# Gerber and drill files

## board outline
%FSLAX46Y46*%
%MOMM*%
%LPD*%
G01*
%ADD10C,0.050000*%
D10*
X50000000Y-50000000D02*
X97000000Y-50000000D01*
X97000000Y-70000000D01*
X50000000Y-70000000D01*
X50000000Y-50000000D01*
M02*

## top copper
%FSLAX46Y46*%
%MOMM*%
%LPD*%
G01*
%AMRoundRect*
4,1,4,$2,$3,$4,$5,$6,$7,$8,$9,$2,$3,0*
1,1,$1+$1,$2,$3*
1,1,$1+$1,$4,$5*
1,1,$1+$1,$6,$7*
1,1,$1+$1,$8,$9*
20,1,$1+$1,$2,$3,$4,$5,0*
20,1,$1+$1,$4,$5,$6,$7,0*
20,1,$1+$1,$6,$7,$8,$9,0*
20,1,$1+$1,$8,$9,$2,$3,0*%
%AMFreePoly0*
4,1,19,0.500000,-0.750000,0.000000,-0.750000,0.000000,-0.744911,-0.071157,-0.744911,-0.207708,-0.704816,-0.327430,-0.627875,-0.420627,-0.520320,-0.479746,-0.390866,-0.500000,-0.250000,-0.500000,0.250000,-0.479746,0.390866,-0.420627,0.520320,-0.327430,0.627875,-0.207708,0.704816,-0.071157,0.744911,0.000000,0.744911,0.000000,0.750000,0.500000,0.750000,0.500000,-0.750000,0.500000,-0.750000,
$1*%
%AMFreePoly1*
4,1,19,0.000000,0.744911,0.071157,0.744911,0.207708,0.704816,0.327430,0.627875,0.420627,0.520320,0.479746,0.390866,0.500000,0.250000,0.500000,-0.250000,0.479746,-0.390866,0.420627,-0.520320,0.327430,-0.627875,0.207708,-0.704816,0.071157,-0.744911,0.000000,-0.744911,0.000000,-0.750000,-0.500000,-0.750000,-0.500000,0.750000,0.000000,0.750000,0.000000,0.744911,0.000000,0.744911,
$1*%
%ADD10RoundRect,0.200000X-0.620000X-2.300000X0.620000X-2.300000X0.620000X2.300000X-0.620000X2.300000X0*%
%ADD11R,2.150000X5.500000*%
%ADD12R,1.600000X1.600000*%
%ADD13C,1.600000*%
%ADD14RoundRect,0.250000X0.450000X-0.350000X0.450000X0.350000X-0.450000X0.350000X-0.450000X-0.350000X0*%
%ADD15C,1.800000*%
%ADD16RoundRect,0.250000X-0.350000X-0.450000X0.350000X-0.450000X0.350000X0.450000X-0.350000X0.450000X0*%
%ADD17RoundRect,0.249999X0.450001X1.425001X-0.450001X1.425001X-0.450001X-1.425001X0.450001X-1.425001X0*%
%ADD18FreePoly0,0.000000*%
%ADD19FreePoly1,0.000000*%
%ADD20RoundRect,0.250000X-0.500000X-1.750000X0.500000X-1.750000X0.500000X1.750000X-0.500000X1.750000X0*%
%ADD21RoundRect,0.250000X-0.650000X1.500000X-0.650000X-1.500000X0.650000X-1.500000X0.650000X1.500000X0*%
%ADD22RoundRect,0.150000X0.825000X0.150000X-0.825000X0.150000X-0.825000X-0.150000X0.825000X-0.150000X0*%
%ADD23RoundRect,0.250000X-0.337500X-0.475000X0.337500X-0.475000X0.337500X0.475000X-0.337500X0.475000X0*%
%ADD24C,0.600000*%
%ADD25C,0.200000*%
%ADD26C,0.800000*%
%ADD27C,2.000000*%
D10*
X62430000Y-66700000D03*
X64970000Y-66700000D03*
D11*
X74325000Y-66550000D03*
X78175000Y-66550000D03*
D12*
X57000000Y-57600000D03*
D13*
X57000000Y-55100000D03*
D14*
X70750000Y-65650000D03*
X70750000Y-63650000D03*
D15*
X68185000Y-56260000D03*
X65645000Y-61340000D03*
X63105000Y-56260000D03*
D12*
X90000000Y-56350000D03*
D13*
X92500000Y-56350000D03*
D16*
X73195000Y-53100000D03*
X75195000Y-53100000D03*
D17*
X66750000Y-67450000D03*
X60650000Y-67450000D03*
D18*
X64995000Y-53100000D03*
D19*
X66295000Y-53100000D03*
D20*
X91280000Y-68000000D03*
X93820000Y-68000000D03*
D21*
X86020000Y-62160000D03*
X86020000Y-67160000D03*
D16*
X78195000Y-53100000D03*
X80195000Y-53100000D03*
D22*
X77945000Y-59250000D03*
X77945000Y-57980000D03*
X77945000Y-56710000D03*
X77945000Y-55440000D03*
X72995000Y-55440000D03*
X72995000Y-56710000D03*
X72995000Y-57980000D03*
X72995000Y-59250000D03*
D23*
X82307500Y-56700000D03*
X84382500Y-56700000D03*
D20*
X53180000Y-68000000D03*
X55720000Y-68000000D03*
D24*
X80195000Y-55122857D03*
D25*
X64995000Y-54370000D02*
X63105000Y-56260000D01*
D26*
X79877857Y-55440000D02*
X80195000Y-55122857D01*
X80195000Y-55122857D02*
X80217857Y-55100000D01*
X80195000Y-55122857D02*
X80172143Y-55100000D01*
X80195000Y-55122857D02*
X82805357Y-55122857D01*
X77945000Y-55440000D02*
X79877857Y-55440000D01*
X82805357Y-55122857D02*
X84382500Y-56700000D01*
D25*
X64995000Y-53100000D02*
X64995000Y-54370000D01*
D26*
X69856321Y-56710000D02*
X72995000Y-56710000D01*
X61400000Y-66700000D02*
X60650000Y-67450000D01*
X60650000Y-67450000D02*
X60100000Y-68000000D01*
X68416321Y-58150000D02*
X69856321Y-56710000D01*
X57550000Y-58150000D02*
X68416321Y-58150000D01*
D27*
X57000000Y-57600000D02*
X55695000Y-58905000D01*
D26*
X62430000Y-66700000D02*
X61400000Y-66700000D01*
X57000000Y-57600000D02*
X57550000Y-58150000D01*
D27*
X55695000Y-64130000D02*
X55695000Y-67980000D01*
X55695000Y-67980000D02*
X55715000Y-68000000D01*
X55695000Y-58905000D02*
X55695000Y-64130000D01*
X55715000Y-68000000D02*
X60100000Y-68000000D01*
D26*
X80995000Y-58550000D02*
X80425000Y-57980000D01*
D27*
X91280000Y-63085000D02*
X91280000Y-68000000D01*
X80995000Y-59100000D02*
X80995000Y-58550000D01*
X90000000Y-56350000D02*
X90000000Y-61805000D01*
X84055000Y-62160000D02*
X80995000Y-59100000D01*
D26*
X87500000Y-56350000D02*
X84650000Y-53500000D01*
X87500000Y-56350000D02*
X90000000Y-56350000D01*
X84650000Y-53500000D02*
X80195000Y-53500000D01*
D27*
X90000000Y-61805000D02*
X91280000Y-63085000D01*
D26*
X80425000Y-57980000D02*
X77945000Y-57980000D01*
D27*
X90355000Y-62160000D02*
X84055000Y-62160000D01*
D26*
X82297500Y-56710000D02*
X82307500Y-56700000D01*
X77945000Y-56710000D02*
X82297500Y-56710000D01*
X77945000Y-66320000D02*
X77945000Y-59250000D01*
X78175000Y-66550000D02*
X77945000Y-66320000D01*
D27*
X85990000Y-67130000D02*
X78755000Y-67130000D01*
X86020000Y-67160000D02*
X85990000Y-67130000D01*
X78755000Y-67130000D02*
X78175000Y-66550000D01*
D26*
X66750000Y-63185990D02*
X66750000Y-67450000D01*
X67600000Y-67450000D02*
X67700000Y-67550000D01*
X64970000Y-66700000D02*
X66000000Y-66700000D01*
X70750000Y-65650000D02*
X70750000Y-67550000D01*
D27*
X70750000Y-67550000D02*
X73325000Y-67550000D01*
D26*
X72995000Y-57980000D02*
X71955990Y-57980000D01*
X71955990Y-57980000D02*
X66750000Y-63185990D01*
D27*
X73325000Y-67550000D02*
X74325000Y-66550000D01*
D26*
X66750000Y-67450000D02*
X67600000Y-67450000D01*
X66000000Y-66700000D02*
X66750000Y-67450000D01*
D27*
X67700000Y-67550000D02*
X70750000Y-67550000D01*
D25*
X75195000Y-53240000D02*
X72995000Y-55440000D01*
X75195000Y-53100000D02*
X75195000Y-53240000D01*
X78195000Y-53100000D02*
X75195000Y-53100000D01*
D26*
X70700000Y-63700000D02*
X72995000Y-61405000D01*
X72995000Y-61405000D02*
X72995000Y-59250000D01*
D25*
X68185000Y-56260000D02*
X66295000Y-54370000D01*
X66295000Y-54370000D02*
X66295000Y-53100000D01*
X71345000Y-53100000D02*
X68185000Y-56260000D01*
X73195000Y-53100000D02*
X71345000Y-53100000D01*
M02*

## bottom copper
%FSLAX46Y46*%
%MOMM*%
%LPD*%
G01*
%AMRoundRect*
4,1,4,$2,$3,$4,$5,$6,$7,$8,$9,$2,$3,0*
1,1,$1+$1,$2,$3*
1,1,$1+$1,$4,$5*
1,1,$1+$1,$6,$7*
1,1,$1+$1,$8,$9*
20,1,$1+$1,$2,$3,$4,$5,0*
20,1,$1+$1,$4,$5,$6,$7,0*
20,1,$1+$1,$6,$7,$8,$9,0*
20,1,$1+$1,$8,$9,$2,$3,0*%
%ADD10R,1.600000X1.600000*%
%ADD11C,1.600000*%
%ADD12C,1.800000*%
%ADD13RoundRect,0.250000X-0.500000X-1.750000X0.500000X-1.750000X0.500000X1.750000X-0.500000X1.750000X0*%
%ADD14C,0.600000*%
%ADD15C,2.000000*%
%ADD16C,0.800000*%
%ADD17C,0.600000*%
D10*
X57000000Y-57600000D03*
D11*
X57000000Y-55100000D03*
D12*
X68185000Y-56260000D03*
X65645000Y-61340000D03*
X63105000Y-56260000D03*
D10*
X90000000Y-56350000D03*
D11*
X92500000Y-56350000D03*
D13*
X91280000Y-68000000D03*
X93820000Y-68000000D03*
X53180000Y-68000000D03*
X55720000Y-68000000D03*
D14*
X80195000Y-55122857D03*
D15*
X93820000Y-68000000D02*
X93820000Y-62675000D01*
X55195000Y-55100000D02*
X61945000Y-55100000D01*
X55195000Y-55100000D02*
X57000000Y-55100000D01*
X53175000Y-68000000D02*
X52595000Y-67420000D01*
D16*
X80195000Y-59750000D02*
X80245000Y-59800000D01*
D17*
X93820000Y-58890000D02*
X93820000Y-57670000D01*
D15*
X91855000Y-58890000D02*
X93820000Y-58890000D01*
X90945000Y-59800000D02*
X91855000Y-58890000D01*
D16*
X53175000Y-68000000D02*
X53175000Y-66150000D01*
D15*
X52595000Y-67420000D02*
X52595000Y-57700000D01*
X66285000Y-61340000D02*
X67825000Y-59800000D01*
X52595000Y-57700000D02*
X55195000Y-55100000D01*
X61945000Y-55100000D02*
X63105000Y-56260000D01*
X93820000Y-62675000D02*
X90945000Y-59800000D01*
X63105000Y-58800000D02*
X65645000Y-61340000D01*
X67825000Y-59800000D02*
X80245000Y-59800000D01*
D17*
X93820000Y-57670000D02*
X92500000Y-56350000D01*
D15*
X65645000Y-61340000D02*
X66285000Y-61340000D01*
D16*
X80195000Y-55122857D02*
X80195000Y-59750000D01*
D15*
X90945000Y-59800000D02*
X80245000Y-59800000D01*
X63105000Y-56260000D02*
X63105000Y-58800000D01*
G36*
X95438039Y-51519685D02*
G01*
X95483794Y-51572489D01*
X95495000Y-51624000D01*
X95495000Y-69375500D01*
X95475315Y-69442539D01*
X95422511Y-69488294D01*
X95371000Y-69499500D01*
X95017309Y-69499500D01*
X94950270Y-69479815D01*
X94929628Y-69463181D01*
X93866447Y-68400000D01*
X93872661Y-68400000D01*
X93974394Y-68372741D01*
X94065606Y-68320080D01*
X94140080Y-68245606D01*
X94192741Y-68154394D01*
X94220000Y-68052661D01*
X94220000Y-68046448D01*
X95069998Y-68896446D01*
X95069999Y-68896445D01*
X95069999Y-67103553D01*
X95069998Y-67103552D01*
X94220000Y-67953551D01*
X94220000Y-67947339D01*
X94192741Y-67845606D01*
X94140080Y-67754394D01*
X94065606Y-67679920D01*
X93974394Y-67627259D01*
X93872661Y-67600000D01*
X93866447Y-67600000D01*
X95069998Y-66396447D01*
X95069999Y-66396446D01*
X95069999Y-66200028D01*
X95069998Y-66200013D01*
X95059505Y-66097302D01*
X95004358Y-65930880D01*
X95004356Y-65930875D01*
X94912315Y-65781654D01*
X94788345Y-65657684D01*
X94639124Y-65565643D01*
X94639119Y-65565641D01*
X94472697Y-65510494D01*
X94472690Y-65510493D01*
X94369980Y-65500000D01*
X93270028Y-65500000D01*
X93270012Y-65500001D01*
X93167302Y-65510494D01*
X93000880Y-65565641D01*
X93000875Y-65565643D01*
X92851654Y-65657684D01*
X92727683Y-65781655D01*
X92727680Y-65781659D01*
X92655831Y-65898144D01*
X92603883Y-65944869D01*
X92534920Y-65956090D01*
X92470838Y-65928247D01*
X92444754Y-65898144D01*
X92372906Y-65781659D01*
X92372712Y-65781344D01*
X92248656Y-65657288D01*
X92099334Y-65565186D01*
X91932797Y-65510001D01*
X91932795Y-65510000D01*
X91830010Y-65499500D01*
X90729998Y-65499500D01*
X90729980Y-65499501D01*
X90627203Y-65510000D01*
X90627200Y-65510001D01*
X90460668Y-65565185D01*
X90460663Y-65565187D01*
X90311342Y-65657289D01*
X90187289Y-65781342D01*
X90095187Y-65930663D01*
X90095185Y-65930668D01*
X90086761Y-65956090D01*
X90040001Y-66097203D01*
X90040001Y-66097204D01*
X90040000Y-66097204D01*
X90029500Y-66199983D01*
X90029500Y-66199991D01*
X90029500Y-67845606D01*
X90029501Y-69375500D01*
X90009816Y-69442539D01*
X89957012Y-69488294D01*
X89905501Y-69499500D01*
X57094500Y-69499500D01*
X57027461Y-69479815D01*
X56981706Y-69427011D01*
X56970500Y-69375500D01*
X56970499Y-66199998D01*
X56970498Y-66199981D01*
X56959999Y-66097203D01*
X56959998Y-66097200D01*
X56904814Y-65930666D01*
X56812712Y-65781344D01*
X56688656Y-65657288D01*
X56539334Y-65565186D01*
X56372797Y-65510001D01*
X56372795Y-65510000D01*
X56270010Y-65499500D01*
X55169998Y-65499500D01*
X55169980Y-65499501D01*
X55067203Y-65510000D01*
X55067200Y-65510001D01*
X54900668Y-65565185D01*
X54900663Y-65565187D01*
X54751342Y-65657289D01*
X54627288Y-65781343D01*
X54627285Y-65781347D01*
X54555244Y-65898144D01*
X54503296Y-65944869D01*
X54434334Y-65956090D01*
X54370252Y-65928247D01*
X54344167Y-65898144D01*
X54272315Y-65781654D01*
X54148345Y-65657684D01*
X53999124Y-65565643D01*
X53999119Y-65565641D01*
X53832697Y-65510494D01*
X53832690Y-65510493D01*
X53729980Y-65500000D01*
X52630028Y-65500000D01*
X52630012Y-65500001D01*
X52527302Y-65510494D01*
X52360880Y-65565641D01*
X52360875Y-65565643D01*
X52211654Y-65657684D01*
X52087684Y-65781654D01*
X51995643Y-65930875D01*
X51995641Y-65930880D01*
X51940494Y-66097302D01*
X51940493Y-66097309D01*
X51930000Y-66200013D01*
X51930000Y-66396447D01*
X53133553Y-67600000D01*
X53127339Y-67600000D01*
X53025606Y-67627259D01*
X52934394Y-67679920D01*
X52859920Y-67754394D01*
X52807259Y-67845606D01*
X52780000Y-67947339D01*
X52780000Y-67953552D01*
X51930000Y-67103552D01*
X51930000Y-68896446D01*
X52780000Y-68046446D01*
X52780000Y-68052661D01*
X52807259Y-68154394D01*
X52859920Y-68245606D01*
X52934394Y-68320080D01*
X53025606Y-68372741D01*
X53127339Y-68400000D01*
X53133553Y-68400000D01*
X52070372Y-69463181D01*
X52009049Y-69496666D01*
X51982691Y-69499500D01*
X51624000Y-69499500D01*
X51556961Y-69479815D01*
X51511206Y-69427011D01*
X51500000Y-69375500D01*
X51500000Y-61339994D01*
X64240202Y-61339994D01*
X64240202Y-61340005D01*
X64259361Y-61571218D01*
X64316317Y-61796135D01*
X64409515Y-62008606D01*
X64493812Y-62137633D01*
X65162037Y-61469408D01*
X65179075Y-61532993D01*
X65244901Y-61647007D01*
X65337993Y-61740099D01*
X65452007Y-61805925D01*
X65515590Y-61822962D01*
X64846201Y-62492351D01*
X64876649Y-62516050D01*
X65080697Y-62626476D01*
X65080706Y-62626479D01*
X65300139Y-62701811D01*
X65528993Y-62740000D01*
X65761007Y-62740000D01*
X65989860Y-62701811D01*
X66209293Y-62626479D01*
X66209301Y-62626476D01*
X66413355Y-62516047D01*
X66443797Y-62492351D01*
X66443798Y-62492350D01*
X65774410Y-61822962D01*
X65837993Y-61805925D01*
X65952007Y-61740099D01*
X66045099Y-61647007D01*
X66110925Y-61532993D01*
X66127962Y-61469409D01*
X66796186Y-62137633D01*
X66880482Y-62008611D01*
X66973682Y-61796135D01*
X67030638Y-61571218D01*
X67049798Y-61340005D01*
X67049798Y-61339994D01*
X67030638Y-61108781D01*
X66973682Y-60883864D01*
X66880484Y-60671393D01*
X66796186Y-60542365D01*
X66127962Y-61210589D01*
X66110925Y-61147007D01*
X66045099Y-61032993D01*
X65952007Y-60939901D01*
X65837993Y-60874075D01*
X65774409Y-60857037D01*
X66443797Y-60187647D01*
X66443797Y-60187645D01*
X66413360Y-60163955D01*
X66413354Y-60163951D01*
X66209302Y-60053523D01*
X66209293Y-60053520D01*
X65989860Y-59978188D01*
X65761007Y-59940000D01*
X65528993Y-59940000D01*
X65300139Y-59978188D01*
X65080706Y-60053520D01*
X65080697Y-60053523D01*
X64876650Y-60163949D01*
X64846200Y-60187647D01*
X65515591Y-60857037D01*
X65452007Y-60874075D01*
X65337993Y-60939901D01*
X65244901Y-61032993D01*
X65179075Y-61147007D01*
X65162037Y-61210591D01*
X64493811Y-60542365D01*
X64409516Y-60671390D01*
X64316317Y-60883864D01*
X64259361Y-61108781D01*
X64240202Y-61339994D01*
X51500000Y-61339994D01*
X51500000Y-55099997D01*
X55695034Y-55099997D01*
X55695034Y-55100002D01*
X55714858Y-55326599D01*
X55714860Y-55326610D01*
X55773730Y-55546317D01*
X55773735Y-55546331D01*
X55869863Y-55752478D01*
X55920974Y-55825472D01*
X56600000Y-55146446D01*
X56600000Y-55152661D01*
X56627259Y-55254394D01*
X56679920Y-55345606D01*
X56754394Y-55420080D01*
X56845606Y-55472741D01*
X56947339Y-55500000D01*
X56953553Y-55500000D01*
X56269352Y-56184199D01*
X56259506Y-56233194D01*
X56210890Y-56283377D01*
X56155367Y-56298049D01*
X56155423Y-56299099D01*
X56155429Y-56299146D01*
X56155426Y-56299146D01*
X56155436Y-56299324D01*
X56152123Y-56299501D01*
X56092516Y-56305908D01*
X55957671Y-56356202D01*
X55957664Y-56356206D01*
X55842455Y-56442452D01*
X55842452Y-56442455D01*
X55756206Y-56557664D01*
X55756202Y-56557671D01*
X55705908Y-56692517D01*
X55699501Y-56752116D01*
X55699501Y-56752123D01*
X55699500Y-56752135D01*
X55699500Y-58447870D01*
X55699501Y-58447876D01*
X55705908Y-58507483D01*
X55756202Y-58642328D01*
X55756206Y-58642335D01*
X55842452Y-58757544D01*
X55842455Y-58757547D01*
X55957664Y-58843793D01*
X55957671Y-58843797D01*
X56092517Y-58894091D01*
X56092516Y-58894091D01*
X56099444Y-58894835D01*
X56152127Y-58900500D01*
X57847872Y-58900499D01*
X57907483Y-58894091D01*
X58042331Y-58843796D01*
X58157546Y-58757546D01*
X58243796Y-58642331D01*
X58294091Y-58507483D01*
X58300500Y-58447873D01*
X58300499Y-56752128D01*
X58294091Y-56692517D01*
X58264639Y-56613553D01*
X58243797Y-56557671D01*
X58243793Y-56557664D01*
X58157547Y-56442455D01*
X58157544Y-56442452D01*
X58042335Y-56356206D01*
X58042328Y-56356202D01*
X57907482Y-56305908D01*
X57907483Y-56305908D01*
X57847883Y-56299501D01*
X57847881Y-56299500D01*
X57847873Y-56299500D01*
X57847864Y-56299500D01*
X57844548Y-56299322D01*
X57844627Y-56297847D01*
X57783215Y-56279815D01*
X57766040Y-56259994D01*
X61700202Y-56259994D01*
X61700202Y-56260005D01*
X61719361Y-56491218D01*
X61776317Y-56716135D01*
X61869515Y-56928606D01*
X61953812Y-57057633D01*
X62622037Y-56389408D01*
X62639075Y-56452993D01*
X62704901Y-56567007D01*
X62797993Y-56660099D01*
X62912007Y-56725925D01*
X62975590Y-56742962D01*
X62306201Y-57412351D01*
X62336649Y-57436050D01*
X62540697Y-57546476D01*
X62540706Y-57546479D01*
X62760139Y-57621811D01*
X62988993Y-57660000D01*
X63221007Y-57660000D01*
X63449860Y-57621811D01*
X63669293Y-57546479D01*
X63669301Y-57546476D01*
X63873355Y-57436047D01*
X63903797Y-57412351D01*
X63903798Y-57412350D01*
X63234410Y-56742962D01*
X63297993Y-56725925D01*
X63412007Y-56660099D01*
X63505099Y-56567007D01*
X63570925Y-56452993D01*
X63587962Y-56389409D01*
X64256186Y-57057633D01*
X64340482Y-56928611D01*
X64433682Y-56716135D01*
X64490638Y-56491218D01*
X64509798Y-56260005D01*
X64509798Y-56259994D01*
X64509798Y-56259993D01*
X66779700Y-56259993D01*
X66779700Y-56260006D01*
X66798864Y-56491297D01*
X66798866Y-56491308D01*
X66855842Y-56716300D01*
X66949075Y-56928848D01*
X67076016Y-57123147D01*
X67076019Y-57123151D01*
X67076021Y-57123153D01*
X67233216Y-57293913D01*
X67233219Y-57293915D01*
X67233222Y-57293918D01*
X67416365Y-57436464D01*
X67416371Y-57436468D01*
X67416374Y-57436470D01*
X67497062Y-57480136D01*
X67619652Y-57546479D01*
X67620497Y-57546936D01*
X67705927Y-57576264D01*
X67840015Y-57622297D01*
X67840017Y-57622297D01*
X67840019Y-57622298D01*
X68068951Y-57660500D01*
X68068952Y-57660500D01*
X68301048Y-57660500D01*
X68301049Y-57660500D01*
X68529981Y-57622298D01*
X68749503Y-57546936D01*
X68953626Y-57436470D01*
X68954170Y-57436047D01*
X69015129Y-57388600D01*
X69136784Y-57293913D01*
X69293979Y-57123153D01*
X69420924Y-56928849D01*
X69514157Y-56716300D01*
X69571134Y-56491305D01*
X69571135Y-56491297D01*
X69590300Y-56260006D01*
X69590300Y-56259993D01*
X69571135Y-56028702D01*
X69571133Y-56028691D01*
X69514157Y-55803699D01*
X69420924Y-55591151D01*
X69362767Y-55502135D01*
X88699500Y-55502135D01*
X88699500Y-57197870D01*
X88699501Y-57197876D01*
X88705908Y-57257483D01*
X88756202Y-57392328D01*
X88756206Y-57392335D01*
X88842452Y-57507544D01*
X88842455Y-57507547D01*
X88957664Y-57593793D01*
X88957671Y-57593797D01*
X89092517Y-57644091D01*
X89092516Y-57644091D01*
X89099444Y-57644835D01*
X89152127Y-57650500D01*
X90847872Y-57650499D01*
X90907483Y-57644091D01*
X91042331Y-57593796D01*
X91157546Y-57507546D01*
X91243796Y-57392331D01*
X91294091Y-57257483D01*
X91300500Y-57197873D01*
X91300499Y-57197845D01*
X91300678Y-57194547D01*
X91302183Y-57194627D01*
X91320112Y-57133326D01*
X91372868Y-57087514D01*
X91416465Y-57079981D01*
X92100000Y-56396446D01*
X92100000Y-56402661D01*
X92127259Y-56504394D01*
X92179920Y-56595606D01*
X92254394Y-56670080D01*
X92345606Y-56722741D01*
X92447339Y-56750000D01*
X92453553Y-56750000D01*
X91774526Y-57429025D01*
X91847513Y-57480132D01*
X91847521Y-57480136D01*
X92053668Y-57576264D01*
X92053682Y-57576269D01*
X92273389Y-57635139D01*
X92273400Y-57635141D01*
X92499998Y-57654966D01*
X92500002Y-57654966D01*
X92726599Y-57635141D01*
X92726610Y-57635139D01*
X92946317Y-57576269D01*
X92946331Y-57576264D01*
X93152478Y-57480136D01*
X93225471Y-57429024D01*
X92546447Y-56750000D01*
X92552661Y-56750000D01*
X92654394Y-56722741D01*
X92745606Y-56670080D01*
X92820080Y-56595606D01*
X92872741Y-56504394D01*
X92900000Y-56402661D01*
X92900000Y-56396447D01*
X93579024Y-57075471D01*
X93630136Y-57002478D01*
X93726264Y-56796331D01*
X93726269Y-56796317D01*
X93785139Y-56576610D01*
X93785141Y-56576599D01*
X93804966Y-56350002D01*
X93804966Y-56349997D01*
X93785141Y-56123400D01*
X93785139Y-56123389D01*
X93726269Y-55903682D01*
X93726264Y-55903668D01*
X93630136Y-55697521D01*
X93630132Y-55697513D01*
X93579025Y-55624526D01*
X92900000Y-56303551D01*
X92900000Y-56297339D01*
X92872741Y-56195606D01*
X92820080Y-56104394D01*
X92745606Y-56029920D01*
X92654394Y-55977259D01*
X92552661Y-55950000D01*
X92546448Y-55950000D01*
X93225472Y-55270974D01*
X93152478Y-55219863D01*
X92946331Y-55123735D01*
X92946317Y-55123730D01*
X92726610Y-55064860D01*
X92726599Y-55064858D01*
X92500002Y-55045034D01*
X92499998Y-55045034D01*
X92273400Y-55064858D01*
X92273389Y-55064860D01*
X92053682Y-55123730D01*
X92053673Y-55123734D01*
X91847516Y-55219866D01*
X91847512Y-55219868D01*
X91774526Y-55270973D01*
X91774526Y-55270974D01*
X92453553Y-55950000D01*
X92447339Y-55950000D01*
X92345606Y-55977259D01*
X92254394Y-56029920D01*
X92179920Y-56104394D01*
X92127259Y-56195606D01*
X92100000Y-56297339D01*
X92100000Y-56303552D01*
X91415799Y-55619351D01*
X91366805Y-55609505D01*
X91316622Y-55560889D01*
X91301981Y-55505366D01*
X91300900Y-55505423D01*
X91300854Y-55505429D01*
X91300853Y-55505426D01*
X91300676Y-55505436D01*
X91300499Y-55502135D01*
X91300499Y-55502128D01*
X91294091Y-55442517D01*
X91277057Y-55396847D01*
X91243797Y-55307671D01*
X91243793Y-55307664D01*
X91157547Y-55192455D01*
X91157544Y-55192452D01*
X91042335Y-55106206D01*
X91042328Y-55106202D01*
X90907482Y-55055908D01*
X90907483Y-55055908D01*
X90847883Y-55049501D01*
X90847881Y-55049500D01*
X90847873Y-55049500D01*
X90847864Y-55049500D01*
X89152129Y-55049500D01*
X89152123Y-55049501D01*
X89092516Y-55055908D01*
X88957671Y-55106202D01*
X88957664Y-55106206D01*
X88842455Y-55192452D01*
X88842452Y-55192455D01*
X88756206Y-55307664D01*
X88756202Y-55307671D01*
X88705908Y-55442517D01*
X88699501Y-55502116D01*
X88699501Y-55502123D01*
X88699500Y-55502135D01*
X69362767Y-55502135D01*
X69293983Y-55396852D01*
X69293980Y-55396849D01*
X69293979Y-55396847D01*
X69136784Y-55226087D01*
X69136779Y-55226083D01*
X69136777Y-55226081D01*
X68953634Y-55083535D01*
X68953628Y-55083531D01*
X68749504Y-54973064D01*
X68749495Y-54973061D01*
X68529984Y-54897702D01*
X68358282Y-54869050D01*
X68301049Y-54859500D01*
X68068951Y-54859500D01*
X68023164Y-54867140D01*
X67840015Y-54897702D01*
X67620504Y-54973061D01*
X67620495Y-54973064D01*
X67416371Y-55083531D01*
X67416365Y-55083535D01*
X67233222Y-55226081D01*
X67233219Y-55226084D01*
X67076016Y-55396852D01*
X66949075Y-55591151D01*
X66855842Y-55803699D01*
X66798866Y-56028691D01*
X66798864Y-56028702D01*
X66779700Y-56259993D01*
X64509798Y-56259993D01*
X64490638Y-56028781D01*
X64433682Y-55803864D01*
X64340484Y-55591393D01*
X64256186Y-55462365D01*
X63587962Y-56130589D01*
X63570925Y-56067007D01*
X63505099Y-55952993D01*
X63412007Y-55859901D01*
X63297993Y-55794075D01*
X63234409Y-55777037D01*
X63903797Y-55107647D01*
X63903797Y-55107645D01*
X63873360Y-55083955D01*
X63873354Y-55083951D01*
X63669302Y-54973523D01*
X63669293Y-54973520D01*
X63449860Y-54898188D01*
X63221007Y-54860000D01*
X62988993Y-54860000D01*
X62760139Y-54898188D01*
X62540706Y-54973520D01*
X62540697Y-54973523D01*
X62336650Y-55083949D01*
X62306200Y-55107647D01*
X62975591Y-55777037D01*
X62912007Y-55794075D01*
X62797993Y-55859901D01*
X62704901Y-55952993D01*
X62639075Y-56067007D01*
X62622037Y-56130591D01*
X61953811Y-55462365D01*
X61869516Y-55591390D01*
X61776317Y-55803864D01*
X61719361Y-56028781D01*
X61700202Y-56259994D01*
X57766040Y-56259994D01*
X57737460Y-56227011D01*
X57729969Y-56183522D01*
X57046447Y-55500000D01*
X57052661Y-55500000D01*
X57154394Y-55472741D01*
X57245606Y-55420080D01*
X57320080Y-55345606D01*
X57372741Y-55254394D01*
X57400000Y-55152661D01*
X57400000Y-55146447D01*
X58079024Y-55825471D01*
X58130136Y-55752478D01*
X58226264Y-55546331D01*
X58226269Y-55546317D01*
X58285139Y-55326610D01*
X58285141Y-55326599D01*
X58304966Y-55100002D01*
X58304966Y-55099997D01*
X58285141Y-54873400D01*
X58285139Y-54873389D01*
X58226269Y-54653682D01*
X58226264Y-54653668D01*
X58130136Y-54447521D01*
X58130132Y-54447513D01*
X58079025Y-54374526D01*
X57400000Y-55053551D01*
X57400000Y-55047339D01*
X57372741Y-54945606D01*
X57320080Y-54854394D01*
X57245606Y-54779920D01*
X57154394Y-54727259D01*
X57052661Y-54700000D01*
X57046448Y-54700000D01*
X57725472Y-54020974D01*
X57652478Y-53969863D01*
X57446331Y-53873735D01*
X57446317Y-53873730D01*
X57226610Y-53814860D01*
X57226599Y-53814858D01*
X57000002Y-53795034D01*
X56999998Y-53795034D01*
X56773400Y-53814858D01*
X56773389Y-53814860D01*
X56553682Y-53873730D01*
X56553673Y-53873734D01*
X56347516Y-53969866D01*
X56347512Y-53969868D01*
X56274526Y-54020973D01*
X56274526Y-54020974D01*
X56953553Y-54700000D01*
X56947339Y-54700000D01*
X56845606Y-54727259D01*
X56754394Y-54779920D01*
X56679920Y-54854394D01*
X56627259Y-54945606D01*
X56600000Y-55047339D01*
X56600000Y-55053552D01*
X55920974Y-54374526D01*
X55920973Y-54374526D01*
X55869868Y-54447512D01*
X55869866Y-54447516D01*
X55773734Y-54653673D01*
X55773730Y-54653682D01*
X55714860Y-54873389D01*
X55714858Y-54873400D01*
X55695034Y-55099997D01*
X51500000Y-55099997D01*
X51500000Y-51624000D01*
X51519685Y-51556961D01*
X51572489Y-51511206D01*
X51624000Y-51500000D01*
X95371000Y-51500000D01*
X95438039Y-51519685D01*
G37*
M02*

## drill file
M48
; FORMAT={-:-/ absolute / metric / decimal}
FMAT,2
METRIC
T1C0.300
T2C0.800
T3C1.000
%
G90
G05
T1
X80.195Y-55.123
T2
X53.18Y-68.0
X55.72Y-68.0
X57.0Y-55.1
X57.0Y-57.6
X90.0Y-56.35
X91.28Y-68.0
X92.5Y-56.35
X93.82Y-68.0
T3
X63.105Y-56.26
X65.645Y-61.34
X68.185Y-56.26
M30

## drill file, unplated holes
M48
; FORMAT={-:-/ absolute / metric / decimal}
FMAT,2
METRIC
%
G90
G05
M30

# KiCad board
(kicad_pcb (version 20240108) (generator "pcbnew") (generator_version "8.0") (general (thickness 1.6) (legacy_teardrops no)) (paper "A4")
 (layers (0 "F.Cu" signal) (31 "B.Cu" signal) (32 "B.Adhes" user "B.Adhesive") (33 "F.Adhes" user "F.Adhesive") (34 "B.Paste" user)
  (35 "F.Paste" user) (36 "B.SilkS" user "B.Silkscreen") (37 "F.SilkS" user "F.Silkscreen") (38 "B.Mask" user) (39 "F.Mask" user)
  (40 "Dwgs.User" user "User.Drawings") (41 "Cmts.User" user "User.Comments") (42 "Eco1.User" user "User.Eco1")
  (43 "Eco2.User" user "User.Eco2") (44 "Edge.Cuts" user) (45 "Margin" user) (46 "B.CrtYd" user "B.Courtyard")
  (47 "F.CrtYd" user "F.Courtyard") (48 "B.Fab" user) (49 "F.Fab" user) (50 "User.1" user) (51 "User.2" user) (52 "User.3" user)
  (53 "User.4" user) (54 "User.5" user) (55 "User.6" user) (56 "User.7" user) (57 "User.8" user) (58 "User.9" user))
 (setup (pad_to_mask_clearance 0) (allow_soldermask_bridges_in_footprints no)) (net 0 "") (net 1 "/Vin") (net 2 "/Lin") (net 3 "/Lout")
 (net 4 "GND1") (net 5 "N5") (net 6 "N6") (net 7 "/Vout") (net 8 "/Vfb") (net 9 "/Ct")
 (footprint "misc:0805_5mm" (layer "F.Cu") (at 63.7 66.7)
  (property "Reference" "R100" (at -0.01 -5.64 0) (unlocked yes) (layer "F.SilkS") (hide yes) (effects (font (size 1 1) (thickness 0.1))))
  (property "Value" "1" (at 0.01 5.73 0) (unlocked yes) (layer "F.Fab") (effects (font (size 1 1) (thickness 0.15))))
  (pad "1" smd roundrect (at -1.27 0) (size 1.64 5) (layers "F.Cu" "F.Paste" "F.Mask") (roundrect_rratio 0.1219512195) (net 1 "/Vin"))
  (pad "2" smd roundrect (at 1.27 0) (size 1.64 5) (layers "F.Cu" "F.Paste" "F.Mask") (roundrect_rratio 0.1219512195) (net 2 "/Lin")))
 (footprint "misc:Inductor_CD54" (layer "F.Cu") (at 76.25 66.55 90)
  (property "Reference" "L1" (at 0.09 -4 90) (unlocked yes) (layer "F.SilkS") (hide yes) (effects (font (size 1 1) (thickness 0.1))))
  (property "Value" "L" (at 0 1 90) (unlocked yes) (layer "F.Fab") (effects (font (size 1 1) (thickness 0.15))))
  (pad "1" smd rect (at 0 -1.925 90) (size 5.5 2.15) (layers "F.Cu" "F.Paste" "F.Mask") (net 2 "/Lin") (thermal_bridge_angle 45))
  (pad "2" smd rect (at 0 1.925 90) (size 5.5 2.15) (layers "F.Cu" "F.Paste" "F.Mask") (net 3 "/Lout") (thermal_bridge_angle 45)))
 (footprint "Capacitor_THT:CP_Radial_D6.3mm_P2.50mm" (layer "F.Cu") (at 57 57.6 90)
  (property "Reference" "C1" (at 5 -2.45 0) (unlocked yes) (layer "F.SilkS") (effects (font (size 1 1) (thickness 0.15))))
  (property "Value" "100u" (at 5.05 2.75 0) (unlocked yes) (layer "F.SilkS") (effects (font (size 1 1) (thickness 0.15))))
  (pad "1" thru_hole rect (at 0 0 90) (size 1.6 1.6) (drill 0.8) (layers "*.Cu" "*.Mask") (remove_unused_layers no) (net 1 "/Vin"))
  (pad "2" thru_hole circle (at 2.5 0 90) (size 1.6 1.6) (drill 0.8) (layers "*.Cu" "*.Mask") (remove_unused_layers no) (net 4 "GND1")))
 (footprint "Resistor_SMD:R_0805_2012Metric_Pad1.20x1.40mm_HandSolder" (layer "F.Cu") (at 70.75 64.65 90)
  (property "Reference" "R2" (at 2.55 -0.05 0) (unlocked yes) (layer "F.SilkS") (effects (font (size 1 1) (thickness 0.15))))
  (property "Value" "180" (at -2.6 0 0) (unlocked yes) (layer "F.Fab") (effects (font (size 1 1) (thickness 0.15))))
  (pad "1" smd roundrect (at -1 0 90) (size 1.2 1.4) (layers "F.Cu" "F.Paste" "F.Mask") (roundrect_rratio 0.208333) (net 2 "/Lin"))
  (pad "2" smd roundrect (at 1 0 90) (size 1.2 1.4) (layers "F.Cu" "F.Paste" "F.Mask") (roundrect_rratio 0.208333) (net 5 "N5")))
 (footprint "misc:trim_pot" (layer "F.Cu") (at 65.645 58.8 180)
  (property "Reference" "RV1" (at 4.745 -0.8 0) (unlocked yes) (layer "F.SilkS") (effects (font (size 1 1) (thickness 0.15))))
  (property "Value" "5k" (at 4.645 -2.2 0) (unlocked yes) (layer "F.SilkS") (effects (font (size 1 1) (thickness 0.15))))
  (pad "1" thru_hole circle (at -2.54 2.54 180) (size 1.8 1.8) (drill 1) (layers "*.Cu" "*.Mask") (remove_unused_layers no) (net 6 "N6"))
  (pad "2" thru_hole circle (at 0 -2.54 180) (size 1.8 1.8) (drill 1) (layers "*.Cu" "*.Mask") (remove_unused_layers no) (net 4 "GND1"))
  (pad "3" thru_hole circle (at 2.54 2.54 180) (size 1.8 1.8) (drill 1) (layers "*.Cu" "*.Mask") (remove_unused_layers no) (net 4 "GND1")))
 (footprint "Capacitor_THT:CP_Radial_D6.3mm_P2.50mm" (layer "F.Cu") (at 90 56.35)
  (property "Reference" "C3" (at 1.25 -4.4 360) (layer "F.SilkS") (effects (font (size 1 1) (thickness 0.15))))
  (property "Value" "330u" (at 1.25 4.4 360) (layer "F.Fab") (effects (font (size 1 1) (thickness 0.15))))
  (pad "1" thru_hole rect (at 0 0) (size 1.6 1.6) (drill 0.8) (layers "*.Cu" "*.Mask") (remove_unused_layers no) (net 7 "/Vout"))
  (pad "2" thru_hole circle (at 2.5 0) (size 1.6 1.6) (drill 0.8) (layers "*.Cu" "*.Mask") (remove_unused_layers no) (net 4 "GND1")))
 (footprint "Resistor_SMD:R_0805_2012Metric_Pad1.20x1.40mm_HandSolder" (layer "F.Cu") (at 74.195 53.1)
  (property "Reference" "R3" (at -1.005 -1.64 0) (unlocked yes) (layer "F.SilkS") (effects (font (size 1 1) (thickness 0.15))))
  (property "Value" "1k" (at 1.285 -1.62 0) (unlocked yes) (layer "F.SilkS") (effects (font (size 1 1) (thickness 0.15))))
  (pad "1" smd roundrect (at -1 0) (size 1.2 1.4) (layers "F.Cu" "F.Paste" "F.Mask") (roundrect_rratio 0.208333) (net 6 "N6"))
  (pad "2" smd roundrect (at 1 0) (size 1.2 1.4) (layers "F.Cu" "F.Paste" "F.Mask") (roundrect_rratio 0.208333) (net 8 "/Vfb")))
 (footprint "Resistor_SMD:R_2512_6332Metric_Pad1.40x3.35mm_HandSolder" (layer "F.Cu") (at 63.7 67.45 180)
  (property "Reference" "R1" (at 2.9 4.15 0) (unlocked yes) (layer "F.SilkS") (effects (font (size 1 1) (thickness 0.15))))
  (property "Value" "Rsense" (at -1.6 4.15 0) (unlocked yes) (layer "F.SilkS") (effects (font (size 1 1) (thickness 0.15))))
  (pad "1" smd roundrect (at -3.05 0 180) (size 1.4 3.35) (layers "F.Cu" "F.Paste" "F.Mask") (roundrect_rratio 0.178571) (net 2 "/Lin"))
  (pad "2" smd roundrect (at 3.05 0 180) (size 1.4 3.35) (layers "F.Cu" "F.Paste" "F.Mask") (roundrect_rratio 0.178571) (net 1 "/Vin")))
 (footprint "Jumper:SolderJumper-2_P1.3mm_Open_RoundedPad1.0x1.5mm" (layer "F.Cu") (at 65.645 53.1)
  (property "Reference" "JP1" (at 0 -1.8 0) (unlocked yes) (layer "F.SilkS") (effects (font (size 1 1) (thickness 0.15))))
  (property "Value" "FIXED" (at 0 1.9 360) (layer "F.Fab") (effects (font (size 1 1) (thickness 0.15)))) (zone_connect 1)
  (pad "1" smd custom (at -0.65 0) (size 1 0.5) (layers "F.Cu" "F.Mask") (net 4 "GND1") (zone_connect 2) (thermal_bridge_angle 45)
   (options (clearance outline) (anchor rect)) (primitives))
  (pad "2" smd custom (at 0.65 0) (size 1 0.5) (layers "F.Cu" "F.Mask") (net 6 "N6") (zone_connect 2) (thermal_bridge_angle 45)
   (options (clearance outline) (anchor rect)) (primitives)))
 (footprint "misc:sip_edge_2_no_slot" (layer "F.Cu") (at 92.55 70)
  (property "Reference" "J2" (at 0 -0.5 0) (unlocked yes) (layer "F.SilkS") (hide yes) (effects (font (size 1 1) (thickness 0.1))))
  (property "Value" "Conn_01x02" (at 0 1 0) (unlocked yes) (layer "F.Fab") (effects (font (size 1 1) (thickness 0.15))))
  (pad "1" thru_hole roundrect (at -1.27 -2) (size 1.5 4) (drill 0.8) (layers "*.Cu" "*.Mask") (remove_unused_layers no)
   (roundrect_rratio 0.1666666667) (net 7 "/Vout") (thermal_bridge_angle 45))
  (pad "2" thru_hole roundrect (at 1.27 -2) (size 1.5 4) (drill 0.8) (layers "*.Cu" "*.Mask") (remove_unused_layers no)
   (roundrect_rratio 0.1666666667) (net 4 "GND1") (thermal_bridge_angle 45)))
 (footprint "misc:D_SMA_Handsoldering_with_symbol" (layer "F.Cu") (at 86.02 64.66 -90)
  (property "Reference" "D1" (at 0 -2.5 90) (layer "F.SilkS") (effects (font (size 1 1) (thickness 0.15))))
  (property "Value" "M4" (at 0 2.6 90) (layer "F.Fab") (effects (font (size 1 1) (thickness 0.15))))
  (pad "1" smd roundrect (at -2.5 0 270) (size 3.5 1.8) (layers "F.Cu" "F.Paste" "F.Mask") (roundrect_rratio 0.1388888889) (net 7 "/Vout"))
  (pad "2" smd roundrect (at 2.5 0 270) (size 3.5 1.8) (layers "F.Cu" "F.Paste" "F.Mask") (roundrect_rratio 0.1388888889) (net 3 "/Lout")))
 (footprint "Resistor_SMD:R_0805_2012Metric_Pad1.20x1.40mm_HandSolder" (layer "F.Cu") (at 79.195 53.1)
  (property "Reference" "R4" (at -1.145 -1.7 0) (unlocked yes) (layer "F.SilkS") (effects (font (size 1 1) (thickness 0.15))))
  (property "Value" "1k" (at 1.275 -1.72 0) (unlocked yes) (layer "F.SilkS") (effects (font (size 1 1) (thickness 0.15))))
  (pad "1" smd roundrect (at -1 0) (size 1.2 1.4) (layers "F.Cu" "F.Paste" "F.Mask") (roundrect_rratio 0.208333) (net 8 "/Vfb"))
  (pad "2" smd roundrect (at 1 0) (size 1.2 1.4) (layers "F.Cu" "F.Paste" "F.Mask") (roundrect_rratio 0.208333) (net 7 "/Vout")))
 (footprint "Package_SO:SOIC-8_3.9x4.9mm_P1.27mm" (layer "F.Cu") (at 75.47 57.345 180)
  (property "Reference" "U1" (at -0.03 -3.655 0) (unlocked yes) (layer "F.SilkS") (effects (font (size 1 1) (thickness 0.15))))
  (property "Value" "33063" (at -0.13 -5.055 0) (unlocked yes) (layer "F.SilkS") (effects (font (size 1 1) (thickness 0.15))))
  (pad "1" smd roundrect (at -2.475 -1.905 180) (size 1.95 0.6) (layers "F.Cu" "F.Paste" "F.Mask") (roundrect_rratio 0.25) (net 3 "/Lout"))
  (pad "2" smd roundrect (at -2.475 -0.635 180) (size 1.95 0.6) (layers "F.Cu" "F.Paste" "F.Mask") (roundrect_rratio 0.25) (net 7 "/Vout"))
  (pad "3" smd roundrect (at -2.475 0.635 180) (size 1.95 0.6) (layers "F.Cu" "F.Paste" "F.Mask") (roundrect_rratio 0.25) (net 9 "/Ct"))
  (pad "4" smd roundrect (at -2.475 1.905 180) (size 1.95 0.6) (layers "F.Cu" "F.Paste" "F.Mask") (roundrect_rratio 0.25) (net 4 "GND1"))
  (pad "5" smd roundrect (at 2.475 1.905 180) (size 1.95 0.6) (layers "F.Cu" "F.Paste" "F.Mask") (roundrect_rratio 0.25) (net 8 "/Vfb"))
  (pad "6" smd roundrect (at 2.475 0.635 180) (size 1.95 0.6) (layers "F.Cu" "F.Paste" "F.Mask") (roundrect_rratio 0.25) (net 1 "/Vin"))
  (pad "7" smd roundrect (at 2.475 -0.635 180) (size 1.95 0.6) (layers "F.Cu" "F.Paste" "F.Mask") (roundrect_rratio 0.25) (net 2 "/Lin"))
  (pad "8" smd roundrect (at 2.475 -1.905 180) (size 1.95 0.6) (layers "F.Cu" "F.Paste" "F.Mask") (roundrect_rratio 0.25) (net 5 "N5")))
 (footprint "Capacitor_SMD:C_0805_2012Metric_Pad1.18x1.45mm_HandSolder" (layer "F.Cu") (at 83.345 56.7)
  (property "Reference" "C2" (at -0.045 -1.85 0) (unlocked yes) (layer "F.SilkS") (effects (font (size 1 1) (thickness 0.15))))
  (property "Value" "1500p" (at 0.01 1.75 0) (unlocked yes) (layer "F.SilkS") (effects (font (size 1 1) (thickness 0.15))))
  (pad "1" smd roundrect (at -1.0375 0) (size 1.175 1.45) (layers "F.Cu" "F.Paste" "F.Mask") (roundrect_rratio 0.212766) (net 9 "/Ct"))
  (pad "2" smd roundrect (at 1.0375 0) (size 1.175 1.45) (layers "F.Cu" "F.Paste" "F.Mask") (roundrect_rratio 0.212766) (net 4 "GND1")))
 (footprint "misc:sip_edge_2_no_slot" (layer "F.Cu") (at 54.45 70)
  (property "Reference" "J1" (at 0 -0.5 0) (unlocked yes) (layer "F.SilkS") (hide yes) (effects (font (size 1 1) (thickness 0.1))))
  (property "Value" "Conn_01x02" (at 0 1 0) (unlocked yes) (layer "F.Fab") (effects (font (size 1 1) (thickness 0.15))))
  (pad "1" thru_hole roundrect (at -1.27 -2) (size 1.5 4) (drill 0.8) (layers "*.Cu" "*.Mask") (remove_unused_layers no)
   (roundrect_rratio 0.1666666667) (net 4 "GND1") (thermal_bridge_angle 45))
  (pad "2" thru_hole roundrect (at 1.27 -2) (size 1.5 4) (drill 0.8) (layers "*.Cu" "*.Mask") (remove_unused_layers no)
   (roundrect_rratio 0.1666666667) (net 1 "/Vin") (thermal_bridge_angle 45)))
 (gr_rect (start 50 50) (end 97 70) (stroke (width 0.05) (type default)) (fill none) (layer "Edge.Cuts"))
 (segment (start 70.7 63.7) (end 72.995 61.405) (width 0.8) (layer "F.Cu") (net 5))
 (segment (start 72.995 61.405) (end 72.995 59.25) (width 0.8) (layer "F.Cu") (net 5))
 (segment (start 64.995 54.37) (end 63.105 56.26) (width 0.2) (layer "F.Cu") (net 4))
 (segment (start 79.877857 55.44) (end 80.195 55.122857) (width 0.8) (layer "F.Cu") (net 4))
 (segment (start 80.195 55.122857) (end 80.217857 55.1) (width 0.8) (layer "F.Cu") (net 4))
 (segment (start 80.195 55.122857) (end 80.172143 55.1) (width 0.8) (layer "F.Cu") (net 4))
 (segment (start 80.195 55.122857) (end 82.805357 55.122857) (width 0.8) (layer "F.Cu") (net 4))
 (segment (start 77.945 55.44) (end 79.877857 55.44) (width 0.8) (layer "F.Cu") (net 4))
 (segment (start 82.805357 55.122857) (end 84.3825 56.7) (width 0.8) (layer "F.Cu") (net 4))
 (segment (start 64.995 53.1) (end 64.995 54.37) (width 0.2) (layer "F.Cu") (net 4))
 (via (at 80.195 55.122857) (size 0.6) (drill 0.3) (layers "F.Cu" "B.Cu") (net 4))
 (segment (start 93.82 68) (end 93.82 62.675) (width 2) (layer "B.Cu") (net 4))
 (segment (start 55.195 55.1) (end 61.945 55.1) (width 2) (layer "B.Cu") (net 4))
 (segment (start 55.195 55.1) (end 57 55.1) (width 2) (layer "B.Cu") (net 4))
 (segment (start 53.175 68) (end 52.595 67.42) (width 2) (layer "B.Cu") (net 4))
 (segment (start 80.195 59.75) (end 80.245 59.8) (width 0.8) (layer "B.Cu") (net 4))
 (segment (start 93.82 58.89) (end 93.82 57.67) (width 0.6) (layer "B.Cu") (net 4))
 (segment (start 91.855 58.89) (end 93.82 58.89) (width 2) (layer "B.Cu") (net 4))
 (segment (start 90.945 59.8) (end 91.855 58.89) (width 2) (layer "B.Cu") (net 4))
 (segment (start 53.175 68) (end 53.175 66.15) (width 0.8) (layer "B.Cu") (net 4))
 (segment (start 52.595 67.42) (end 52.595 57.7) (width 2) (layer "B.Cu") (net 4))
 (segment (start 66.285 61.34) (end 67.825 59.8) (width 2) (layer "B.Cu") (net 4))
 (segment (start 52.595 57.7) (end 55.195 55.1) (width 2) (layer "B.Cu") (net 4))
 (segment (start 61.945 55.1) (end 63.105 56.26) (width 2) (layer "B.Cu") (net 4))
 (segment (start 93.82 62.675) (end 90.945 59.8) (width 2) (layer "B.Cu") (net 4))
 (segment (start 63.105 58.8) (end 65.645 61.34) (width 2) (layer "B.Cu") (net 4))
 (segment (start 67.825 59.8) (end 80.245 59.8) (width 2) (layer "B.Cu") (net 4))
 (segment (start 93.82 57.67) (end 92.5 56.35) (width 0.6) (layer "B.Cu") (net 4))
 (segment (start 65.645 61.34) (end 66.285 61.34) (width 2) (layer "B.Cu") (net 4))
 (segment (start 80.195 55.122857) (end 80.195 59.75) (width 0.8) (layer "B.Cu") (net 4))
 (segment (start 90.945 59.8) (end 80.245 59.8) (width 2) (layer "B.Cu") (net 4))
 (segment (start 63.105 56.26) (end 63.105 58.8) (width 2) (layer "B.Cu") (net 4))
 (segment (start 69.856321 56.71) (end 72.995 56.71) (width 0.8) (layer "F.Cu") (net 1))
 (segment (start 61.4 66.7) (end 60.65 67.45) (width 0.8) (layer "F.Cu") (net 1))
 (segment (start 60.65 67.45) (end 60.1 68) (width 0.8) (layer "F.Cu") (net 1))
 (segment (start 68.416321 58.15) (end 69.856321 56.71) (width 0.8) (layer "F.Cu") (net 1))
 (segment (start 57.55 58.15) (end 68.416321 58.15) (width 0.8) (layer "F.Cu") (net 1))
 (segment (start 57 57.6) (end 55.695 58.905) (width 2) (layer "F.Cu") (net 1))
 (segment (start 62.43 66.7) (end 61.4 66.7) (width 0.8) (layer "F.Cu") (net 1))
 (segment (start 57 57.6) (end 57.55 58.15) (width 0.8) (layer "F.Cu") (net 1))
 (segment (start 55.695 64.13) (end 55.695 67.98) (width 2) (layer "F.Cu") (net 1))
 (segment (start 55.695 67.98) (end 55.715 68) (width 2) (layer "F.Cu") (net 1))
 (segment (start 55.695 58.905) (end 55.695 64.13) (width 2) (layer "F.Cu") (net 1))
 (segment (start 55.715 68) (end 60.1 68) (width 2) (layer "F.Cu") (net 1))
 (segment (start 80.995 58.55) (end 80.425 57.98) (width 0.8) (layer "F.Cu") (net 7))
 (segment (start 91.28 63.085) (end 91.28 68) (width 2) (layer "F.Cu") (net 7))
 (segment (start 80.995 59.1) (end 80.995 58.55) (width 2) (layer "F.Cu") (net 7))
 (segment (start 90 56.35) (end 90 61.805) (width 2) (layer "F.Cu") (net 7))
 (segment (start 84.055 62.16) (end 80.995 59.1) (width 2) (layer "F.Cu") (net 7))
 (segment (start 87.5 56.35) (end 84.65 53.5) (width 0.8) (layer "F.Cu") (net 7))
 (segment (start 87.5 56.35) (end 90 56.35) (width 0.8) (layer "F.Cu") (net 7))
 (segment (start 84.65 53.5) (end 80.195 53.5) (width 0.8) (layer "F.Cu") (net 7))
 (segment (start 90 61.805) (end 91.28 63.085) (width 2) (layer "F.Cu") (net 7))
 (segment (start 80.425 57.98) (end 77.945 57.98) (width 0.8) (layer "F.Cu") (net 7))
 (segment (start 90.355 62.16) (end 84.055 62.16) (width 2) (layer "F.Cu") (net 7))
 (segment (start 82.2975 56.71) (end 82.3075 56.7) (width 0.8) (layer "F.Cu") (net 9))
 (segment (start 77.945 56.71) (end 82.2975 56.71) (width 0.8) (layer "F.Cu") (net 9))
 (segment (start 77.945 66.32) (end 77.945 59.25) (width 0.8) (layer "F.Cu") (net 3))
 (segment (start 78.175 66.55) (end 77.945 66.32) (width 0.8) (layer "F.Cu") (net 3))
 (segment (start 85.99 67.13) (end 78.755 67.13) (width 2) (layer "F.Cu") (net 3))
 (segment (start 86.02 67.16) (end 85.99 67.13) (width 2) (layer "F.Cu") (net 3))
 (segment (start 78.755 67.13) (end 78.175 66.55) (width 2) (layer "F.Cu") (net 3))
 (segment (start 66.75 63.18599) (end 66.75 67.45) (width 0.8) (layer "F.Cu") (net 2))
 (segment (start 67.6 67.45) (end 67.7 67.55) (width 0.8) (layer "F.Cu") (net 2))
 (segment (start 64.97 66.7) (end 66 66.7) (width 0.8) (layer "F.Cu") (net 2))
 (segment (start 70.75 65.65) (end 70.75 67.55) (width 0.8) (layer "F.Cu") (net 2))
 (segment (start 70.75 67.55) (end 73.325 67.55) (width 2) (layer "F.Cu") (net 2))
 (segment (start 72.995 57.98) (end 71.95599 57.98) (width 0.8) (layer "F.Cu") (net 2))
 (segment (start 71.95599 57.98) (end 66.75 63.18599) (width 0.8) (layer "F.Cu") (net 2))
 (segment (start 73.325 67.55) (end 74.325 66.55) (width 2) (layer "F.Cu") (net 2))
 (segment (start 66.75 67.45) (end 67.6 67.45) (width 0.8) (layer "F.Cu") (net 2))
 (segment (start 66 66.7) (end 66.75 67.45) (width 0.8) (layer "F.Cu") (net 2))
 (segment (start 67.7 67.55) (end 70.75 67.55) (width 2) (layer "F.Cu") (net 2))
 (segment (start 75.195 53.24) (end 72.995 55.44) (width 0.2) (layer "F.Cu") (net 8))
 (segment (start 75.195 53.1) (end 75.195 53.24) (width 0.2) (layer "F.Cu") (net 8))
 (segment (start 78.195 53.1) (end 75.195 53.1) (width 0.2) (layer "F.Cu") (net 8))
 (segment (start 68.185 56.26) (end 66.295 54.37) (width 0.2) (layer "F.Cu") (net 6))
 (segment (start 66.295 54.37) (end 66.295 53.1) (width 0.2) (layer "F.Cu") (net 6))
 (segment (start 71.345 53.1) (end 68.185 56.26) (width 0.2) (layer "F.Cu") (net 6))
 (segment (start 73.195 53.1) (end 71.345 53.1) (width 0.2) (layer "F.Cu") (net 6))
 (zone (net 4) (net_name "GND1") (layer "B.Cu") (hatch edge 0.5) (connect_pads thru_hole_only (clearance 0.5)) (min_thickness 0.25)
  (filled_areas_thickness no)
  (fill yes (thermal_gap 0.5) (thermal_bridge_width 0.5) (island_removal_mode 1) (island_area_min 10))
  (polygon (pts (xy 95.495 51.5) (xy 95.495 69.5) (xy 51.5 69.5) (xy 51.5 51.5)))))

